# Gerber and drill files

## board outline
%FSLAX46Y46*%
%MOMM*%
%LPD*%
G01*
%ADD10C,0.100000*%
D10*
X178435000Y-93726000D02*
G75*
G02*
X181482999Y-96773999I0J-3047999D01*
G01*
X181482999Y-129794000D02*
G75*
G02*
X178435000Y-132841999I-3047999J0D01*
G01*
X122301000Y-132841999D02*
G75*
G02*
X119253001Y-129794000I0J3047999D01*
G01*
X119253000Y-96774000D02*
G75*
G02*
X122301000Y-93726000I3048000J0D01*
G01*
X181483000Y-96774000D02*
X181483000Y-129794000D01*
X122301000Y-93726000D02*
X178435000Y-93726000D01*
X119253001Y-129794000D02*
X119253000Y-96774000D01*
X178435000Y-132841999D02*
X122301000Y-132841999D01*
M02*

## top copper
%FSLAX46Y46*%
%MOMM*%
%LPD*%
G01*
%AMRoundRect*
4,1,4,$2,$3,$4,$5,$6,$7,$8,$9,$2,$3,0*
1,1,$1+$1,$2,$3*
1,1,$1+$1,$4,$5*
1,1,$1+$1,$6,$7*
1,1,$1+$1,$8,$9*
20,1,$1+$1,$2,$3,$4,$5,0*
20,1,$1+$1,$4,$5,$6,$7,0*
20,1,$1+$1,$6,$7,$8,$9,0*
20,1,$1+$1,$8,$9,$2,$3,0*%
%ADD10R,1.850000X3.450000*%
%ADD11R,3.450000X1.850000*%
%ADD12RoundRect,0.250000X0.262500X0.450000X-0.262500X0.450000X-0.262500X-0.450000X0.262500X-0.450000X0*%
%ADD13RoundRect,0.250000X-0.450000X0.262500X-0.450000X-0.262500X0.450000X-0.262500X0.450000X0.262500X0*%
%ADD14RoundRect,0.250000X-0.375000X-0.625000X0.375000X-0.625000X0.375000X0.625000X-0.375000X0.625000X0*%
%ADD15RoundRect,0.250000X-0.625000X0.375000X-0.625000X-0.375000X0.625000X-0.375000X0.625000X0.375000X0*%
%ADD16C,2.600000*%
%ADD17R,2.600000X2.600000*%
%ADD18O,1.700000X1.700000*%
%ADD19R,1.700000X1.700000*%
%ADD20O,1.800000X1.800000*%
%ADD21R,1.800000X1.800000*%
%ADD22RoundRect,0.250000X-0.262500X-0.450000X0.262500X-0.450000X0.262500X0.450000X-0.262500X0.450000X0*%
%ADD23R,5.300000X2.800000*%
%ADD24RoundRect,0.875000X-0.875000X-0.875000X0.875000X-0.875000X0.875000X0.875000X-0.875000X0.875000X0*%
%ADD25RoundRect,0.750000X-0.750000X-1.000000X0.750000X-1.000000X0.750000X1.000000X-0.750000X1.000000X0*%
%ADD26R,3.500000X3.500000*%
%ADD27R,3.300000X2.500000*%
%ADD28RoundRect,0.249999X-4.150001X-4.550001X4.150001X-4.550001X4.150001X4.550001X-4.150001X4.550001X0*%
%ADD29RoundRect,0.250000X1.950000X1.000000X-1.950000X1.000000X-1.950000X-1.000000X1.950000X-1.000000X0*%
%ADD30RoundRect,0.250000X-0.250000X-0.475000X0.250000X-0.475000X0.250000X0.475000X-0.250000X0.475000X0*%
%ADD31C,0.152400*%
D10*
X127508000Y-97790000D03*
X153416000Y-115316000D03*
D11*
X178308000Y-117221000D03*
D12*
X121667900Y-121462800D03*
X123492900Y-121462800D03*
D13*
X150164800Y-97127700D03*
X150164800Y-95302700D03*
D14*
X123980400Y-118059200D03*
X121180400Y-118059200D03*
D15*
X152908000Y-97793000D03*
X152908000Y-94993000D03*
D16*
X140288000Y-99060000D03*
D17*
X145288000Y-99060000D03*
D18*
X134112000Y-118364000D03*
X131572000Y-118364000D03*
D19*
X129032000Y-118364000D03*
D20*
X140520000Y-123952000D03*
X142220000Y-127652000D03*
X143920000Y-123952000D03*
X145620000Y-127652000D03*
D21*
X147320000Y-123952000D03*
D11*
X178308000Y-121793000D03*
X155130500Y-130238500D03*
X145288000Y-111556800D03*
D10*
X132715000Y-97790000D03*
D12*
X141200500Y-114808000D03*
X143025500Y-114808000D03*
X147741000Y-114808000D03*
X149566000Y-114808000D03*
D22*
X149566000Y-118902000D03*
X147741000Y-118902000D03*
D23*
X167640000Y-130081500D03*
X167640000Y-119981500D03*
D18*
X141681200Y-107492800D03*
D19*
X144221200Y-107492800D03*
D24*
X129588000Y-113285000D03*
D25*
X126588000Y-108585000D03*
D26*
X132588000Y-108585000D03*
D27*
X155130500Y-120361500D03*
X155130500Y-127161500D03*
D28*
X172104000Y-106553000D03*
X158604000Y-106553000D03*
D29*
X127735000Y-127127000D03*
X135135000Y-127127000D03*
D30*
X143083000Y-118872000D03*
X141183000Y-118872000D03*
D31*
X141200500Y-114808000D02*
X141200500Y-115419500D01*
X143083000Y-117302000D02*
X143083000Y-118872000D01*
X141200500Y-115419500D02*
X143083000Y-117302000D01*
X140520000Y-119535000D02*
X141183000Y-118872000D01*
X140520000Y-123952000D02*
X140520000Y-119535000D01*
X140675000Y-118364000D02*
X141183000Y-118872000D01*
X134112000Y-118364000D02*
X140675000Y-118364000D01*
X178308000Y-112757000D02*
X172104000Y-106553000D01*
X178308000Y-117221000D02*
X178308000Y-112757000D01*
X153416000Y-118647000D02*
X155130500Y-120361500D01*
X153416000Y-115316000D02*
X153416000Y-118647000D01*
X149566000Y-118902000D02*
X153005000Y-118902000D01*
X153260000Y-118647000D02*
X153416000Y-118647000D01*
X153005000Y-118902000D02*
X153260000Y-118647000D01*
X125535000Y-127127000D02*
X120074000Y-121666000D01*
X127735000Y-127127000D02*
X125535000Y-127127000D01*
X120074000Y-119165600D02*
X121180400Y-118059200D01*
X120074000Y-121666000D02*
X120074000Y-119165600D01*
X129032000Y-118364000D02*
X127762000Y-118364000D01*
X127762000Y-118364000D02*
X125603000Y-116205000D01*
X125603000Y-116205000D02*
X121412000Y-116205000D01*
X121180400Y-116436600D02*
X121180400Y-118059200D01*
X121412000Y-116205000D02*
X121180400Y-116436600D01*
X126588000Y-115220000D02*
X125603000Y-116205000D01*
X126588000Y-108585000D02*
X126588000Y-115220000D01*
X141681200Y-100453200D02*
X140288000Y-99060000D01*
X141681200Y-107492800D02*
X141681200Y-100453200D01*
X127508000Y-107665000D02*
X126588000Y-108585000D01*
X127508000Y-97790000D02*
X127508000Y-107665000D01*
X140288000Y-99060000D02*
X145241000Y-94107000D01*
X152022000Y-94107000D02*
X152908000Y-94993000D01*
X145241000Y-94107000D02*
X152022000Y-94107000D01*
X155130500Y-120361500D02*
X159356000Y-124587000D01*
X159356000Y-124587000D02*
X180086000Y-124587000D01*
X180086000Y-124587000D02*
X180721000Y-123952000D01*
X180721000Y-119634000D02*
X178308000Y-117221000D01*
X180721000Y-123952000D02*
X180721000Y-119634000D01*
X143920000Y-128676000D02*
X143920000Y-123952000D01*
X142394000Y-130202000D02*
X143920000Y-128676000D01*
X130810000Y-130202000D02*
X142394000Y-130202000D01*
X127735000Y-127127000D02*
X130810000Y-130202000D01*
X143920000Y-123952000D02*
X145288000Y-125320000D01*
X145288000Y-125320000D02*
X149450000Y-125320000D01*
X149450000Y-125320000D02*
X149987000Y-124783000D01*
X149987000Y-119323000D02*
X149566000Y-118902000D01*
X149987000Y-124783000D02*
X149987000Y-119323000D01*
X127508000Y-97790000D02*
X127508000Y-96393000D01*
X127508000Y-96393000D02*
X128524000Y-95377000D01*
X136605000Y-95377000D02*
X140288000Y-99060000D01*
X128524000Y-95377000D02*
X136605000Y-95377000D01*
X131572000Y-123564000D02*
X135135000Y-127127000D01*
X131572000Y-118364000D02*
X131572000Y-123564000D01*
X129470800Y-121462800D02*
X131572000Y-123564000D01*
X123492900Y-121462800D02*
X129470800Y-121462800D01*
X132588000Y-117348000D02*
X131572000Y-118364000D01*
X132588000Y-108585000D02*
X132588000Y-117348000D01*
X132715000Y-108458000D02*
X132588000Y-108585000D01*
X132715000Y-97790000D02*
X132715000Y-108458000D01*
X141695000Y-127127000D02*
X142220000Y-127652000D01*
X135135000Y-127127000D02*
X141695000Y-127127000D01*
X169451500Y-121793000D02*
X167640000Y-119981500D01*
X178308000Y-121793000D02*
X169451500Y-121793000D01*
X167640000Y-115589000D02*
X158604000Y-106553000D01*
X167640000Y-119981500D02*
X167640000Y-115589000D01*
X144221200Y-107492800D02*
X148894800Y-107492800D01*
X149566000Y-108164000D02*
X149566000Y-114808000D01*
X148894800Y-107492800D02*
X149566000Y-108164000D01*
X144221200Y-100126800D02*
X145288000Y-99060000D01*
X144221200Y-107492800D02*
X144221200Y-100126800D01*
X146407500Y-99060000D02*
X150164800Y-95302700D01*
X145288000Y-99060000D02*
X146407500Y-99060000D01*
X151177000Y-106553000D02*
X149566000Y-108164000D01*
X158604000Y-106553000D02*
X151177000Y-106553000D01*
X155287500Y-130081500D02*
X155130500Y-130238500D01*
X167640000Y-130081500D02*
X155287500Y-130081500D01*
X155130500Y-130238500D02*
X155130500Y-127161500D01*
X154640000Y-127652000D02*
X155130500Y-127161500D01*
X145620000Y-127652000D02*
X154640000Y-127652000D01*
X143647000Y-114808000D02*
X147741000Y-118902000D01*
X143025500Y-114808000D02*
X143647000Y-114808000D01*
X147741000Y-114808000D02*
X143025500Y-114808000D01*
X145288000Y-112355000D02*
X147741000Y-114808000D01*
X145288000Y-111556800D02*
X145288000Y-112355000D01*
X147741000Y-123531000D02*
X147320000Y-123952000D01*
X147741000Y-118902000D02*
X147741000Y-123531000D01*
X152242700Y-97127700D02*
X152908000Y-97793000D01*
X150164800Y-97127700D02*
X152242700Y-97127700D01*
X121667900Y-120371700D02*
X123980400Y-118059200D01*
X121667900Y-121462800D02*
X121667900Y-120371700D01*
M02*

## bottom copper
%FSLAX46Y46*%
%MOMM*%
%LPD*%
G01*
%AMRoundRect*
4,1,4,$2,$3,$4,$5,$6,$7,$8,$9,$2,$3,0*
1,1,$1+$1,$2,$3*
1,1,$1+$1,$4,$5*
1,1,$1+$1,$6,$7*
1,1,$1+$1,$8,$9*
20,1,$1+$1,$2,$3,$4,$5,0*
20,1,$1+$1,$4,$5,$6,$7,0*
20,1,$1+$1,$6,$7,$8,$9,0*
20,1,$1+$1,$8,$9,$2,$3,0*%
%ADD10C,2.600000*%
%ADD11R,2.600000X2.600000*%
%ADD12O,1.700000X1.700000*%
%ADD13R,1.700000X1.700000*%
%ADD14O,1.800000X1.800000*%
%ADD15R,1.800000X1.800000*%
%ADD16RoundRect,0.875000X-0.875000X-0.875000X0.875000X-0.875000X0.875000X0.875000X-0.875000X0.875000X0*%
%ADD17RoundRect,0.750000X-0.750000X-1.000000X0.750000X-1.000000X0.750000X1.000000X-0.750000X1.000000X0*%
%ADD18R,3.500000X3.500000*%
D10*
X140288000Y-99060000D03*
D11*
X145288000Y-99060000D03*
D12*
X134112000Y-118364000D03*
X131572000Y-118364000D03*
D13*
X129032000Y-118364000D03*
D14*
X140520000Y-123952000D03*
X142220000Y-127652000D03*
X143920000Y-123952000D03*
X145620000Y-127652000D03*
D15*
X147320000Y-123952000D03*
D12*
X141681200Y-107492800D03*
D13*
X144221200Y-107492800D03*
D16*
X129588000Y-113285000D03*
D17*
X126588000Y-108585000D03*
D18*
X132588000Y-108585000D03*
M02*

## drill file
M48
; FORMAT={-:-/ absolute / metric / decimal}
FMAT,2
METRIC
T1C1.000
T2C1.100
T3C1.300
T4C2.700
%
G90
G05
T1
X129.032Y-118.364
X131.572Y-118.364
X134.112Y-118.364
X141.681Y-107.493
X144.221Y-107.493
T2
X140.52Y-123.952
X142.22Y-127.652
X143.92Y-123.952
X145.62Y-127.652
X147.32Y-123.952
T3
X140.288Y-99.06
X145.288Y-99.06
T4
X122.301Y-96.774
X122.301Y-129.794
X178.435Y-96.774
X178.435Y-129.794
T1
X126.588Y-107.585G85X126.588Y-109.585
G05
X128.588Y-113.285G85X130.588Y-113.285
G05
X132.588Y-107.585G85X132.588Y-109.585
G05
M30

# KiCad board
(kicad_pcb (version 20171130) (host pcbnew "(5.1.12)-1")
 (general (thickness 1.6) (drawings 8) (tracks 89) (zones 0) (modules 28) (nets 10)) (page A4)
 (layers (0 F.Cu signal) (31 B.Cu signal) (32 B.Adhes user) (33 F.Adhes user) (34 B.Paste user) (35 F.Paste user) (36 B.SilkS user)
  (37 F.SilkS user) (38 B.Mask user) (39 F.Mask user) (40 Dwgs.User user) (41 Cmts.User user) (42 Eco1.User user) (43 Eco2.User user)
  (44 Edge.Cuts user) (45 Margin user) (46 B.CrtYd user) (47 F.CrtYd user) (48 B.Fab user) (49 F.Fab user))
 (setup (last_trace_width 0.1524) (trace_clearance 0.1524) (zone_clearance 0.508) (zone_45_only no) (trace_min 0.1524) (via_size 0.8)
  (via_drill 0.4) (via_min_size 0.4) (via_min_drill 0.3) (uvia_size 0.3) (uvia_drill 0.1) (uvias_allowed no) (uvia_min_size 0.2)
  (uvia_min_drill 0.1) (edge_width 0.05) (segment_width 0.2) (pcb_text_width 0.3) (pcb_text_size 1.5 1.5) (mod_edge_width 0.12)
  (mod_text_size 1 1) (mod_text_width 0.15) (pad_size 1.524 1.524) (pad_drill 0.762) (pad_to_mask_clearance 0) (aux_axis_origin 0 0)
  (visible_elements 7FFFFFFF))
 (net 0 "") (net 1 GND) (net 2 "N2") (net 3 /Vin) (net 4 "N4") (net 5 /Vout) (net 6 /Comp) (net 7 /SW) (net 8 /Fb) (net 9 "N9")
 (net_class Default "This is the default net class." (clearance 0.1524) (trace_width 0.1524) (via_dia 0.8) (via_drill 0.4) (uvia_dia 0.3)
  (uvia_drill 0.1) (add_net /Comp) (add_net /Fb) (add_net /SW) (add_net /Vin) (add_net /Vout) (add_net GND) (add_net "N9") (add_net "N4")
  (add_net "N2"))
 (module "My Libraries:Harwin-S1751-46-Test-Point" (layer F.Cu) (at 127.508 97.79 90)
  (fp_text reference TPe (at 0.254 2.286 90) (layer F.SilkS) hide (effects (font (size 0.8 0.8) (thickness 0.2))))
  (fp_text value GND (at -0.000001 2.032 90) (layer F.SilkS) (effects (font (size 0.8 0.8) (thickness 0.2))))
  (pad 1 smd rect (at 0 0 90) (size 3.45 1.85) (layers F.Cu F.Paste F.Mask) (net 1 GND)))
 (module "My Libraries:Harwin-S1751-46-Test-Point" (layer F.Cu) (at 153.416 115.316 90)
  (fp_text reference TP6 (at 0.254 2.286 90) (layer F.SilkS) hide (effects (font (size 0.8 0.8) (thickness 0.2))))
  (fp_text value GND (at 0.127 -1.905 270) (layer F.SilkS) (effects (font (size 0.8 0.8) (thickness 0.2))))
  (pad 1 smd rect (at 0 0 90) (size 3.45 1.85) (layers F.Cu F.Paste F.Mask) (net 1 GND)))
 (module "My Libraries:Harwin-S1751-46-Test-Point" (layer F.Cu) (at 178.308 117.221)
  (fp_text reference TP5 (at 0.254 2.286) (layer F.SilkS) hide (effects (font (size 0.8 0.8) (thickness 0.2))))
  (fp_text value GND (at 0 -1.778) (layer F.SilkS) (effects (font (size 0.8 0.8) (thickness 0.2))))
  (pad 1 smd rect (at 0 0) (size 3.45 1.85) (layers F.Cu F.Paste F.Mask) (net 1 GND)))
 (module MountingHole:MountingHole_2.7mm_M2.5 (layer F.Cu) (at 178.435 96.774)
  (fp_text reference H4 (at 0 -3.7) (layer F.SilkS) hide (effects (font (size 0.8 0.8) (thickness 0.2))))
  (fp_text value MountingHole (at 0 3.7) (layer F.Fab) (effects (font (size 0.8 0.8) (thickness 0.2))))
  (pad 1 np_thru_hole circle (at 0 0) (size 2.7 2.7) (drill 2.7) (layers *.Cu *.Mask)))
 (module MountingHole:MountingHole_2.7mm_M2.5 (layer F.Cu) (at 122.301 129.794)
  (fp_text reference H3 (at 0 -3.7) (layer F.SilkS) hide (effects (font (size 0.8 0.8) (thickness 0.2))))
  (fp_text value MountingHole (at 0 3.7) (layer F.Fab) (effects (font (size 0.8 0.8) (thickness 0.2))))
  (pad 1 np_thru_hole circle (at 0 0) (size 2.7 2.7) (drill 2.7) (layers *.Cu *.Mask)))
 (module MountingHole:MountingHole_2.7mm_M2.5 (layer F.Cu) (at 178.435 129.794)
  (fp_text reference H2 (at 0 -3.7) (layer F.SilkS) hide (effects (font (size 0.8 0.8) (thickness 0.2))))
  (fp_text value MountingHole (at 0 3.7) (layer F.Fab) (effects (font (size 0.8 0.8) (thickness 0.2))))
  (pad 1 np_thru_hole circle (at 0 0) (size 2.7 2.7) (drill 2.7) (layers *.Cu *.Mask)))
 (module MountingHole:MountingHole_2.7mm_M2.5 (layer F.Cu) (at 122.301 96.774)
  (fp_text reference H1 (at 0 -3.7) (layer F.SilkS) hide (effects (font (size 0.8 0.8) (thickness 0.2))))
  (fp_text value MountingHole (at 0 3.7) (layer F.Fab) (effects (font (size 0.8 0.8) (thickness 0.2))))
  (pad 1 np_thru_hole circle (at 0 0) (size 2.7 2.7) (drill 2.7) (layers *.Cu *.Mask)))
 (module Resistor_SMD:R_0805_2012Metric (layer F.Cu) (at 122.5804 121.4628 180)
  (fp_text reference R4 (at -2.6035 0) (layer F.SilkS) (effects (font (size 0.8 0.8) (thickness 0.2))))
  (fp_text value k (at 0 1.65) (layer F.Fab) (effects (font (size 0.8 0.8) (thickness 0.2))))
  (pad 2 smd roundrect (at 0.9125 0 180) (size 1.025 1.4) (layers F.Cu F.Paste F.Mask) (roundrect_rratio 0.243902) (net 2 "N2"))
  (pad 1 smd roundrect (at -0.9125 0 180) (size 1.025 1.4) (layers F.Cu F.Paste F.Mask) (roundrect_rratio 0.243902) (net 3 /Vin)))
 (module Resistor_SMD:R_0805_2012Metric (layer F.Cu) (at 150.1648 96.2152 270)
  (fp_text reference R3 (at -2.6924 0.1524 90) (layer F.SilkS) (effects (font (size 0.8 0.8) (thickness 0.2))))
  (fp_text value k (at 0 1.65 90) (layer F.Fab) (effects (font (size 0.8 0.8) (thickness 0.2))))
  (pad 2 smd roundrect (at 0.9125 0 270) (size 1.025 1.4) (layers F.Cu F.Paste F.Mask) (roundrect_rratio 0.243902) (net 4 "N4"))
  (pad 1 smd roundrect (at -0.9125 0 270) (size 1.025 1.4) (layers F.Cu F.Paste F.Mask) (roundrect_rratio 0.243902) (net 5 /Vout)))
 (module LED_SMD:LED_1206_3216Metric (layer F.Cu) (at 122.5804 118.0592)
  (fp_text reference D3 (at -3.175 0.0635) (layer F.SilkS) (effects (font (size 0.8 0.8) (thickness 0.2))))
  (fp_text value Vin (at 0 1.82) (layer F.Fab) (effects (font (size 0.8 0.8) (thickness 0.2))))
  (pad 2 smd roundrect (at 1.4 0) (size 1.25 1.75) (layers F.Cu F.Paste F.Mask) (roundrect_rratio 0.2) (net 2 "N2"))
  (pad 1 smd roundrect (at -1.4 0) (size 1.25 1.75) (layers F.Cu F.Paste F.Mask) (roundrect_rratio 0.2) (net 1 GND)))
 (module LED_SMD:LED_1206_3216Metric (layer F.Cu) (at 152.908 96.393 270)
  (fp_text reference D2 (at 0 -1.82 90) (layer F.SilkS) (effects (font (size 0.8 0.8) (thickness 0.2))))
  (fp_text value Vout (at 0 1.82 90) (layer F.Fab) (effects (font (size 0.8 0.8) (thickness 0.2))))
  (pad 2 smd roundrect (at 1.4 0 270) (size 1.25 1.75) (layers F.Cu F.Paste F.Mask) (roundrect_rratio 0.2) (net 4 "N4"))
  (pad 1 smd roundrect (at -1.4 0 270) (size 1.25 1.75) (layers F.Cu F.Paste F.Mask) (roundrect_rratio 0.2) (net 1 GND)))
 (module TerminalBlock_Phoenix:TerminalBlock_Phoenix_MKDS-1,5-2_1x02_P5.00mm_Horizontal (layer F.Cu) (at 145.288 99.06 180)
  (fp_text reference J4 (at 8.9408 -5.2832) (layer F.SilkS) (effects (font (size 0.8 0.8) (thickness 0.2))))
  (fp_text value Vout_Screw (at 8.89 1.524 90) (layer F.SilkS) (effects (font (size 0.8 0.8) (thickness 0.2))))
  (pad 2 thru_hole circle (at 5 0 180) (size 2.6 2.6) (drill 1.3) (layers *.Cu *.Mask) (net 1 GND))
  (pad 1 thru_hole rect (at 0 0 180) (size 2.6 2.6) (drill 1.3) (layers *.Cu *.Mask) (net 5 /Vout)))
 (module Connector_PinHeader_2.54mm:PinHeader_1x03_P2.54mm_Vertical (layer F.Cu) (at 129.032 118.364 90)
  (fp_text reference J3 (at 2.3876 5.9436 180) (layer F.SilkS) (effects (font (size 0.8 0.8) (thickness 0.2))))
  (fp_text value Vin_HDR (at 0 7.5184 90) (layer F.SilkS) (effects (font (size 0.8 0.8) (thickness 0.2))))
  (pad 3 thru_hole oval (at 0 5.08 90) (size 1.7 1.7) (drill 1) (layers *.Cu *.Mask) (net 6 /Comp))
  (pad 2 thru_hole oval (at 0 2.54 90) (size 1.7 1.7) (drill 1) (layers *.Cu *.Mask) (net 3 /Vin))
  (pad 1 thru_hole rect (at 0 0 90) (size 1.7 1.7) (drill 1) (layers *.Cu *.Mask) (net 1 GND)))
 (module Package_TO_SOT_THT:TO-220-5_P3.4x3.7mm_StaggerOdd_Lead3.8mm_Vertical (layer F.Cu) (at 147.32 123.952 180)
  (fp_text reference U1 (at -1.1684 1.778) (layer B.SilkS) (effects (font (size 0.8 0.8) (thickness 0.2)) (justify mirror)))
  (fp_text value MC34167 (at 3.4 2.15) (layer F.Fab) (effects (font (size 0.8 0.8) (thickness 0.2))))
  (pad 5 thru_hole oval (at 6.8 0 180) (size 1.8 1.8) (drill 1.1) (layers *.Cu *.Mask) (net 6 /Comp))
  (pad 4 thru_hole oval (at 5.1 -3.7 180) (size 1.8 1.8) (drill 1.1) (layers *.Cu *.Mask) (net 3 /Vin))
  (pad 3 thru_hole oval (at 3.4 0 180) (size 1.8 1.8) (drill 1.1) (layers *.Cu *.Mask) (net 1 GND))
  (pad 2 thru_hole oval (at 1.7 -3.7 180) (size 1.8 1.8) (drill 1.1) (layers *.Cu *.Mask) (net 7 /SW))
  (pad 1 thru_hole rect (at 0 0 180) (size 1.8 1.8) (drill 1.1) (layers *.Cu *.Mask) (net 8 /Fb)))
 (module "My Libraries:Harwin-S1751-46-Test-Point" (layer F.Cu) (at 178.308 121.793 180)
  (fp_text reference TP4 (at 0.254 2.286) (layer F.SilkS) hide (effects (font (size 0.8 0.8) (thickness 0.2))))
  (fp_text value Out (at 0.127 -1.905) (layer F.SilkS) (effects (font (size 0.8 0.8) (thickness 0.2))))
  (pad 1 smd rect (at 0 0 180) (size 3.45 1.85) (layers F.Cu F.Paste F.Mask) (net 5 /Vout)))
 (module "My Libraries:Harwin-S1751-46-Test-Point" (layer F.Cu) (at 155.1305 130.2385)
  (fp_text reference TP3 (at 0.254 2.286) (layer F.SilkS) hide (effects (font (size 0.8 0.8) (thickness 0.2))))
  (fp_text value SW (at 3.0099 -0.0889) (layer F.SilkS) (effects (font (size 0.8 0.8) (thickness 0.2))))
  (pad 1 smd rect (at 0 0) (size 3.45 1.85) (layers F.Cu F.Paste F.Mask) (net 7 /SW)))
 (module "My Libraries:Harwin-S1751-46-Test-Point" (layer F.Cu) (at 145.288 111.5568)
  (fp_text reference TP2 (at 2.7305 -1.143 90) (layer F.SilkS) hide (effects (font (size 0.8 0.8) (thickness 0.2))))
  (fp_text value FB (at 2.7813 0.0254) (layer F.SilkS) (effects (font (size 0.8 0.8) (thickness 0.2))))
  (pad 1 smd rect (at 0 0) (size 3.45 1.85) (layers F.Cu F.Paste F.Mask) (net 8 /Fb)))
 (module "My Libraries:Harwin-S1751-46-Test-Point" (layer F.Cu) (at 132.715 97.79 270)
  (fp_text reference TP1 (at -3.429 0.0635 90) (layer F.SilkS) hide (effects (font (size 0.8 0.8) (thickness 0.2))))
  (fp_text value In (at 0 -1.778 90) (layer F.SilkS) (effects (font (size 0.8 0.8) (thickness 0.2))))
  (pad 1 smd rect (at 0 0 270) (size 3.45 1.85) (layers F.Cu F.Paste F.Mask) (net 3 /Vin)))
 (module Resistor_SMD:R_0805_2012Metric (layer F.Cu) (at 142.113 114.808 180)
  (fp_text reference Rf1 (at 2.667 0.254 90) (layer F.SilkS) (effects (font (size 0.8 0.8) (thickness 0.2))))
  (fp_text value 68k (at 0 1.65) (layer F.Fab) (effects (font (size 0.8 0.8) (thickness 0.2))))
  (pad 2 smd roundrect (at 0.9125 0 180) (size 1.025 1.4) (layers F.Cu F.Paste F.Mask) (roundrect_rratio 0.243902) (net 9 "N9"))
  (pad 1 smd roundrect (at -0.9125 0 180) (size 1.025 1.4) (layers F.Cu F.Paste F.Mask) (roundrect_rratio 0.243902) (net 8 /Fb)))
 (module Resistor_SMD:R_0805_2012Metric (layer F.Cu) (at 148.6535 114.808 180)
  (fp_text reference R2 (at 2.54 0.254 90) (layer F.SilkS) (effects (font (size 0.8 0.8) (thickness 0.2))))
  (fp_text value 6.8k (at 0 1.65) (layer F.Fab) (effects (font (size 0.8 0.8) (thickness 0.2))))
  (pad 2 smd roundrect (at 0.9125 0 180) (size 1.025 1.4) (layers F.Cu F.Paste F.Mask) (roundrect_rratio 0.243902) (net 8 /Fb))
  (pad 1 smd roundrect (at -0.9125 0 180) (size 1.025 1.4) (layers F.Cu F.Paste F.Mask) (roundrect_rratio 0.243902) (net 5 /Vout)))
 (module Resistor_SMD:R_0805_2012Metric (layer F.Cu) (at 148.6535 118.902)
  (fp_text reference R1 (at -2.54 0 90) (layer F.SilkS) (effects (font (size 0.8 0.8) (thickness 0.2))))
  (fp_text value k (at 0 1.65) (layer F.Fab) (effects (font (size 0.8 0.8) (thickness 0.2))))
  (pad 2 smd roundrect (at 0.9125 0) (size 1.025 1.4) (layers F.Cu F.Paste F.Mask) (roundrect_rratio 0.243902) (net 1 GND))
  (pad 1 smd roundrect (at -0.9125 0) (size 1.025 1.4) (layers F.Cu F.Paste F.Mask) (roundrect_rratio 0.243902) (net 8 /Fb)))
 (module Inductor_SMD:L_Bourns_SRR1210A (layer F.Cu) (at 167.64 125.0315 90)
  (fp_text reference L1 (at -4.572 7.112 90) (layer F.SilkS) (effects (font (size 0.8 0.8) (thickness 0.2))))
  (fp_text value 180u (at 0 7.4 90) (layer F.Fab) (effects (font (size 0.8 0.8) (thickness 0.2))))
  (pad 1 smd rect (at -5.05 0 90) (size 2.8 5.3) (layers F.Cu F.Paste F.Mask) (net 7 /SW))
  (pad 2 smd rect (at 5.05 0 90) (size 2.8 5.3) (layers F.Cu F.Paste F.Mask) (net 5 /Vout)))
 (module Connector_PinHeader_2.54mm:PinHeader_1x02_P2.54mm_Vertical (layer F.Cu) (at 144.2212 107.4928 270)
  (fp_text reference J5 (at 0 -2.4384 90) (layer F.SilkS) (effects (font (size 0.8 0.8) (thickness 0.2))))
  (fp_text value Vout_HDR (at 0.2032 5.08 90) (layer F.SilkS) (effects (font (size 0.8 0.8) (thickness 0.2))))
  (pad 2 thru_hole oval (at 0 2.54 270) (size 1.7 1.7) (drill 1) (layers *.Cu *.Mask) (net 1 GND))
  (pad 1 thru_hole rect (at 0 0 270) (size 1.7 1.7) (drill 1) (layers *.Cu *.Mask) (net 5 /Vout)))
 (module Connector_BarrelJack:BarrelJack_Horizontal (layer F.Cu) (at 132.588 108.585)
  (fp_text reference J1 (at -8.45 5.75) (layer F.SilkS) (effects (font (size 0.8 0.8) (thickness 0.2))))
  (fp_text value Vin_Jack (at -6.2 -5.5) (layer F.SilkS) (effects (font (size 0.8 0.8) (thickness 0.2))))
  (pad 3 thru_hole roundrect (at -3 4.7) (size 3.5 3.5) (drill oval 3 1) (layers *.Cu *.Mask) (roundrect_rratio 0.25))
  (pad 2 thru_hole roundrect (at -6 0) (size 3 3.5) (drill oval 1 3) (layers *.Cu *.Mask) (roundrect_rratio 0.25) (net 1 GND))
  (pad 1 thru_hole rect (at 0 0) (size 3.5 3.5) (drill oval 1 3) (layers *.Cu *.Mask) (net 3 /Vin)))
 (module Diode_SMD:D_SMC (layer F.Cu) (at 155.1305 123.7615 90)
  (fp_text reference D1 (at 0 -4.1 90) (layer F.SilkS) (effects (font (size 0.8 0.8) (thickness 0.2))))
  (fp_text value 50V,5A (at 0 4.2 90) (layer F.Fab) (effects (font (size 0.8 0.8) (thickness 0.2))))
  (pad 2 smd rect (at 3.4 0 180) (size 3.3 2.5) (layers F.Cu F.Paste F.Mask) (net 1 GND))
  (pad 1 smd rect (at -3.4 0 180) (size 3.3 2.5) (layers F.Cu F.Paste F.Mask) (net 7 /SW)))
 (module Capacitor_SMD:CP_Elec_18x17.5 (layer F.Cu) (at 165.354 106.553)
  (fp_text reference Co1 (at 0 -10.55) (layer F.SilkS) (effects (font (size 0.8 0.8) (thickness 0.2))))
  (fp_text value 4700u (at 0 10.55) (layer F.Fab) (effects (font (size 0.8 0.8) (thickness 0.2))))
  (pad 2 smd roundrect (at 6.75 0) (size 8.8 9.6) (layers F.Cu F.Paste F.Mask) (roundrect_rratio 0.028409) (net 1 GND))
  (pad 1 smd roundrect (at -6.75 0) (size 8.8 9.6) (layers F.Cu F.Paste F.Mask) (roundrect_rratio 0.028409) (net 5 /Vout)))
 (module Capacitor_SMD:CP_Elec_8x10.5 (layer F.Cu) (at 131.435 127.127 180)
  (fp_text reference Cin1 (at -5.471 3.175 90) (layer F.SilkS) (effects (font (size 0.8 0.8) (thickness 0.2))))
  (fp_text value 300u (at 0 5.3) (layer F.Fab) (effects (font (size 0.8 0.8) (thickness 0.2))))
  (pad 2 smd roundrect (at 3.7 0 180) (size 4.4 2.5) (layers F.Cu F.Paste F.Mask) (roundrect_rratio 0.1) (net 1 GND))
  (pad 1 smd roundrect (at -3.7 0 180) (size 4.4 2.5) (layers F.Cu F.Paste F.Mask) (roundrect_rratio 0.1) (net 3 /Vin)))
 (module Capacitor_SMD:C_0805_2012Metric (layer F.Cu) (at 142.133 118.872)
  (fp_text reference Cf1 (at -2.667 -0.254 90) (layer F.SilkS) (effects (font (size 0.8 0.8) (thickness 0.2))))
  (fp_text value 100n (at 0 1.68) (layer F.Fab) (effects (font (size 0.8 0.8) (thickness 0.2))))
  (pad 2 smd roundrect (at 0.95 0) (size 1 1.45) (layers F.Cu F.Paste F.Mask) (roundrect_rratio 0.25) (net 9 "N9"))
  (pad 1 smd roundrect (at -0.95 0) (size 1 1.45) (layers F.Cu F.Paste F.Mask) (roundrect_rratio 0.25) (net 6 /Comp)))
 (gr_arc (start 178.435 96.773999) (end 181.482999 96.773999) (angle -90) (layer Edge.Cuts) (width 0.1))
 (gr_arc (start 178.435 129.794) (end 178.435 132.841999) (angle -90) (layer Edge.Cuts) (width 0.1))
 (gr_arc (start 122.301 129.794) (end 119.253001 129.794) (angle -90) (layer Edge.Cuts) (width 0.1))
 (gr_arc (start 122.301 96.774) (end 122.301 93.726) (angle -90) (layer Edge.Cuts) (width 0.1))
 (gr_line (start 181.483 96.774) (end 181.483 129.794) (layer Edge.Cuts) (width 0.1))
 (gr_line (start 122.301 93.726) (end 178.435 93.726) (layer Edge.Cuts) (width 0.1))
 (gr_line (start 119.253001 129.794) (end 119.253 96.774) (layer Edge.Cuts) (width 0.1))
 (gr_line (start 178.435 132.841999) (end 122.301 132.841999) (layer Edge.Cuts) (width 0.1))
 (segment (start 141.2005 114.808) (end 141.2005 115.4195) (width 0.1524) (layer F.Cu) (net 9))
 (segment (start 143.083 117.302) (end 143.083 118.872) (width 0.1524) (layer F.Cu) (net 9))
 (segment (start 141.2005 115.4195) (end 143.083 117.302) (width 0.1524) (layer F.Cu) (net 9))
 (segment (start 140.52 119.535) (end 141.183 118.872) (width 0.1524) (layer F.Cu) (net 6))
 (segment (start 140.52 123.952) (end 140.52 119.535) (width 0.1524) (layer F.Cu) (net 6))
 (segment (start 140.675 118.364) (end 141.183 118.872) (width 0.1524) (layer F.Cu) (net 6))
 (segment (start 134.112 118.364) (end 140.675 118.364) (width 0.1524) (layer F.Cu) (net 6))
 (segment (start 178.308 112.757) (end 172.104 106.553) (width 0.1524) (layer F.Cu) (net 1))
 (segment (start 178.308 117.221) (end 178.308 112.757) (width 0.1524) (layer F.Cu) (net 1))
 (segment (start 153.416 118.647) (end 155.1305 120.3615) (width 0.1524) (layer F.Cu) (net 1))
 (segment (start 153.416 115.316) (end 153.416 118.647) (width 0.1524) (layer F.Cu) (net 1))
 (segment (start 149.566 118.902) (end 153.005 118.902) (width 0.1524) (layer F.Cu) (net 1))
 (segment (start 153.26 118.647) (end 153.416 118.647) (width 0.1524) (layer F.Cu) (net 1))
 (segment (start 153.005 118.902) (end 153.26 118.647) (width 0.1524) (layer F.Cu) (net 1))
 (segment (start 125.535 127.127) (end 120.074 121.666) (width 0.1524) (layer F.Cu) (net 1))
 (segment (start 127.735 127.127) (end 125.535 127.127) (width 0.1524) (layer F.Cu) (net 1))
 (segment (start 120.074 119.1656) (end 121.1804 118.0592) (width 0.1524) (layer F.Cu) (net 1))
 (segment (start 120.074 121.666) (end 120.074 119.1656) (width 0.1524) (layer F.Cu) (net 1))
 (segment (start 129.032 118.364) (end 127.762 118.364) (width 0.1524) (layer F.Cu) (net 1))
 (segment (start 127.762 118.364) (end 125.603 116.205) (width 0.1524) (layer F.Cu) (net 1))
 (segment (start 125.603 116.205) (end 121.412 116.205) (width 0.1524) (layer F.Cu) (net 1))
 (segment (start 121.1804 116.4366) (end 121.1804 118.0592) (width 0.1524) (layer F.Cu) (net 1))
 (segment (start 121.412 116.205) (end 121.1804 116.4366) (width 0.1524) (layer F.Cu) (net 1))
 (segment (start 126.588 115.22) (end 125.603 116.205) (width 0.1524) (layer F.Cu) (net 1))
 (segment (start 126.588 108.585) (end 126.588 115.22) (width 0.1524) (layer F.Cu) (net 1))
 (segment (start 141.6812 100.4532) (end 140.288 99.06) (width 0.1524) (layer F.Cu) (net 1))
 (segment (start 141.6812 107.4928) (end 141.6812 100.4532) (width 0.1524) (layer F.Cu) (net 1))
 (segment (start 127.508 107.665) (end 126.588 108.585) (width 0.1524) (layer F.Cu) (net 1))
 (segment (start 127.508 97.79) (end 127.508 107.665) (width 0.1524) (layer F.Cu) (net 1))
 (segment (start 140.288 99.06) (end 145.241 94.107) (width 0.1524) (layer F.Cu) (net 1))
 (segment (start 152.022 94.107) (end 152.908 94.993) (width 0.1524) (layer F.Cu) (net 1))
 (segment (start 145.241 94.107) (end 152.022 94.107) (width 0.1524) (layer F.Cu) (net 1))
 (segment (start 155.1305 120.3615) (end 159.356 124.587) (width 0.1524) (layer F.Cu) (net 1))
 (segment (start 159.356 124.587) (end 180.086 124.587) (width 0.1524) (layer F.Cu) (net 1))
 (segment (start 180.086 124.587) (end 180.721 123.952) (width 0.1524) (layer F.Cu) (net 1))
 (segment (start 180.721 119.634) (end 178.308 117.221) (width 0.1524) (layer F.Cu) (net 1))
 (segment (start 180.721 123.952) (end 180.721 119.634) (width 0.1524) (layer F.Cu) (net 1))
 (segment (start 143.92 128.676) (end 143.92 123.952) (width 0.1524) (layer F.Cu) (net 1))
 (segment (start 142.394 130.202) (end 143.92 128.676) (width 0.1524) (layer F.Cu) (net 1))
 (segment (start 130.81 130.202) (end 142.394 130.202) (width 0.1524) (layer F.Cu) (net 1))
 (segment (start 127.735 127.127) (end 130.81 130.202) (width 0.1524) (layer F.Cu) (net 1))
 (segment (start 143.92 123.952) (end 145.288 125.32) (width 0.1524) (layer F.Cu) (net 1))
 (segment (start 145.288 125.32) (end 149.45 125.32) (width 0.1524) (layer F.Cu) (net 1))
 (segment (start 149.45 125.32) (end 149.987 124.783) (width 0.1524) (layer F.Cu) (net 1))
 (segment (start 149.987 119.323) (end 149.566 118.902) (width 0.1524) (layer F.Cu) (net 1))
 (segment (start 149.987 124.783) (end 149.987 119.323) (width 0.1524) (layer F.Cu) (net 1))
 (segment (start 127.508 97.79) (end 127.508 96.393) (width 0.1524) (layer F.Cu) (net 1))
 (segment (start 127.508 96.393) (end 128.524 95.377) (width 0.1524) (layer F.Cu) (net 1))
 (segment (start 136.605 95.377) (end 140.288 99.06) (width 0.1524) (layer F.Cu) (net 1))
 (segment (start 128.524 95.377) (end 136.605 95.377) (width 0.1524) (layer F.Cu) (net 1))
 (segment (start 131.572 123.564) (end 135.135 127.127) (width 0.1524) (layer F.Cu) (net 3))
 (segment (start 131.572 118.364) (end 131.572 123.564) (width 0.1524) (layer F.Cu) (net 3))
 (segment (start 129.4708 121.4628) (end 131.572 123.564) (width 0.1524) (layer F.Cu) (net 3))
 (segment (start 123.4929 121.4628) (end 129.4708 121.4628) (width 0.1524) (layer F.Cu) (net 3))
 (segment (start 132.588 117.348) (end 131.572 118.364) (width 0.1524) (layer F.Cu) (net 3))
 (segment (start 132.588 108.585) (end 132.588 117.348) (width 0.1524) (layer F.Cu) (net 3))
 (segment (start 132.715 108.458) (end 132.588 108.585) (width 0.1524) (layer F.Cu) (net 3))
 (segment (start 132.715 97.79) (end 132.715 108.458) (width 0.1524) (layer F.Cu) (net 3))
 (segment (start 141.695 127.127) (end 142.22 127.652) (width 0.1524) (layer F.Cu) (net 3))
 (segment (start 135.135 127.127) (end 141.695 127.127) (width 0.1524) (layer F.Cu) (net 3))
 (segment (start 169.4515 121.793) (end 167.64 119.9815) (width 0.1524) (layer F.Cu) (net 5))
 (segment (start 178.308 121.793) (end 169.4515 121.793) (width 0.1524) (layer F.Cu) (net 5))
 (segment (start 167.64 115.589) (end 158.604 106.553) (width 0.1524) (layer F.Cu) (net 5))
 (segment (start 167.64 119.9815) (end 167.64 115.589) (width 0.1524) (layer F.Cu) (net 5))
 (segment (start 144.2212 107.4928) (end 148.8948 107.4928) (width 0.1524) (layer F.Cu) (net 5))
 (segment (start 149.566 108.164) (end 149.566 114.808) (width 0.1524) (layer F.Cu) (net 5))
 (segment (start 148.8948 107.4928) (end 149.566 108.164) (width 0.1524) (layer F.Cu) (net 5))
 (segment (start 144.2212 100.1268) (end 145.288 99.06) (width 0.1524) (layer F.Cu) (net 5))
 (segment (start 144.2212 107.4928) (end 144.2212 100.1268) (width 0.1524) (layer F.Cu) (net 5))
 (segment (start 146.4075 99.06) (end 150.1648 95.3027) (width 0.1524) (layer F.Cu) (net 5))
 (segment (start 145.288 99.06) (end 146.4075 99.06) (width 0.1524) (layer F.Cu) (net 5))
 (segment (start 151.177 106.553) (end 149.566 108.164) (width 0.1524) (layer F.Cu) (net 5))
 (segment (start 158.604 106.553) (end 151.177 106.553) (width 0.1524) (layer F.Cu) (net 5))
 (segment (start 155.2875 130.0815) (end 155.1305 130.2385) (width 0.1524) (layer F.Cu) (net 7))
 (segment (start 167.64 130.0815) (end 155.2875 130.0815) (width 0.1524) (layer F.Cu) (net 7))
 (segment (start 155.1305 130.2385) (end 155.1305 127.1615) (width 0.1524) (layer F.Cu) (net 7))
 (segment (start 154.64 127.652) (end 155.1305 127.1615) (width 0.1524) (layer F.Cu) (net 7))
 (segment (start 145.62 127.652) (end 154.64 127.652) (width 0.1524) (layer F.Cu) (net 7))
 (segment (start 143.647 114.808) (end 147.741 118.902) (width 0.1524) (layer F.Cu) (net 8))
 (segment (start 143.0255 114.808) (end 143.647 114.808) (width 0.1524) (layer F.Cu) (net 8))
 (segment (start 147.741 114.808) (end 143.0255 114.808) (width 0.1524) (layer F.Cu) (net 8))
 (segment (start 145.288 112.355) (end 147.741 114.808) (width 0.1524) (layer F.Cu) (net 8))
 (segment (start 145.288 111.5568) (end 145.288 112.355) (width 0.1524) (layer F.Cu) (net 8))
 (segment (start 147.741 123.531) (end 147.32 123.952) (width 0.1524) (layer F.Cu) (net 8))
 (segment (start 147.741 118.902) (end 147.741 123.531) (width 0.1524) (layer F.Cu) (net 8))
 (segment (start 152.2427 97.1277) (end 152.908 97.793) (width 0.1524) (layer F.Cu) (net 4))
 (segment (start 150.1648 97.1277) (end 152.2427 97.1277) (width 0.1524) (layer F.Cu) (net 4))
 (segment (start 121.6679 120.3717) (end 123.9804 118.0592) (width 0.1524) (layer F.Cu) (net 2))
 (segment (start 121.6679 121.4628) (end 121.6679 120.3717) (width 0.1524) (layer F.Cu) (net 2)))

